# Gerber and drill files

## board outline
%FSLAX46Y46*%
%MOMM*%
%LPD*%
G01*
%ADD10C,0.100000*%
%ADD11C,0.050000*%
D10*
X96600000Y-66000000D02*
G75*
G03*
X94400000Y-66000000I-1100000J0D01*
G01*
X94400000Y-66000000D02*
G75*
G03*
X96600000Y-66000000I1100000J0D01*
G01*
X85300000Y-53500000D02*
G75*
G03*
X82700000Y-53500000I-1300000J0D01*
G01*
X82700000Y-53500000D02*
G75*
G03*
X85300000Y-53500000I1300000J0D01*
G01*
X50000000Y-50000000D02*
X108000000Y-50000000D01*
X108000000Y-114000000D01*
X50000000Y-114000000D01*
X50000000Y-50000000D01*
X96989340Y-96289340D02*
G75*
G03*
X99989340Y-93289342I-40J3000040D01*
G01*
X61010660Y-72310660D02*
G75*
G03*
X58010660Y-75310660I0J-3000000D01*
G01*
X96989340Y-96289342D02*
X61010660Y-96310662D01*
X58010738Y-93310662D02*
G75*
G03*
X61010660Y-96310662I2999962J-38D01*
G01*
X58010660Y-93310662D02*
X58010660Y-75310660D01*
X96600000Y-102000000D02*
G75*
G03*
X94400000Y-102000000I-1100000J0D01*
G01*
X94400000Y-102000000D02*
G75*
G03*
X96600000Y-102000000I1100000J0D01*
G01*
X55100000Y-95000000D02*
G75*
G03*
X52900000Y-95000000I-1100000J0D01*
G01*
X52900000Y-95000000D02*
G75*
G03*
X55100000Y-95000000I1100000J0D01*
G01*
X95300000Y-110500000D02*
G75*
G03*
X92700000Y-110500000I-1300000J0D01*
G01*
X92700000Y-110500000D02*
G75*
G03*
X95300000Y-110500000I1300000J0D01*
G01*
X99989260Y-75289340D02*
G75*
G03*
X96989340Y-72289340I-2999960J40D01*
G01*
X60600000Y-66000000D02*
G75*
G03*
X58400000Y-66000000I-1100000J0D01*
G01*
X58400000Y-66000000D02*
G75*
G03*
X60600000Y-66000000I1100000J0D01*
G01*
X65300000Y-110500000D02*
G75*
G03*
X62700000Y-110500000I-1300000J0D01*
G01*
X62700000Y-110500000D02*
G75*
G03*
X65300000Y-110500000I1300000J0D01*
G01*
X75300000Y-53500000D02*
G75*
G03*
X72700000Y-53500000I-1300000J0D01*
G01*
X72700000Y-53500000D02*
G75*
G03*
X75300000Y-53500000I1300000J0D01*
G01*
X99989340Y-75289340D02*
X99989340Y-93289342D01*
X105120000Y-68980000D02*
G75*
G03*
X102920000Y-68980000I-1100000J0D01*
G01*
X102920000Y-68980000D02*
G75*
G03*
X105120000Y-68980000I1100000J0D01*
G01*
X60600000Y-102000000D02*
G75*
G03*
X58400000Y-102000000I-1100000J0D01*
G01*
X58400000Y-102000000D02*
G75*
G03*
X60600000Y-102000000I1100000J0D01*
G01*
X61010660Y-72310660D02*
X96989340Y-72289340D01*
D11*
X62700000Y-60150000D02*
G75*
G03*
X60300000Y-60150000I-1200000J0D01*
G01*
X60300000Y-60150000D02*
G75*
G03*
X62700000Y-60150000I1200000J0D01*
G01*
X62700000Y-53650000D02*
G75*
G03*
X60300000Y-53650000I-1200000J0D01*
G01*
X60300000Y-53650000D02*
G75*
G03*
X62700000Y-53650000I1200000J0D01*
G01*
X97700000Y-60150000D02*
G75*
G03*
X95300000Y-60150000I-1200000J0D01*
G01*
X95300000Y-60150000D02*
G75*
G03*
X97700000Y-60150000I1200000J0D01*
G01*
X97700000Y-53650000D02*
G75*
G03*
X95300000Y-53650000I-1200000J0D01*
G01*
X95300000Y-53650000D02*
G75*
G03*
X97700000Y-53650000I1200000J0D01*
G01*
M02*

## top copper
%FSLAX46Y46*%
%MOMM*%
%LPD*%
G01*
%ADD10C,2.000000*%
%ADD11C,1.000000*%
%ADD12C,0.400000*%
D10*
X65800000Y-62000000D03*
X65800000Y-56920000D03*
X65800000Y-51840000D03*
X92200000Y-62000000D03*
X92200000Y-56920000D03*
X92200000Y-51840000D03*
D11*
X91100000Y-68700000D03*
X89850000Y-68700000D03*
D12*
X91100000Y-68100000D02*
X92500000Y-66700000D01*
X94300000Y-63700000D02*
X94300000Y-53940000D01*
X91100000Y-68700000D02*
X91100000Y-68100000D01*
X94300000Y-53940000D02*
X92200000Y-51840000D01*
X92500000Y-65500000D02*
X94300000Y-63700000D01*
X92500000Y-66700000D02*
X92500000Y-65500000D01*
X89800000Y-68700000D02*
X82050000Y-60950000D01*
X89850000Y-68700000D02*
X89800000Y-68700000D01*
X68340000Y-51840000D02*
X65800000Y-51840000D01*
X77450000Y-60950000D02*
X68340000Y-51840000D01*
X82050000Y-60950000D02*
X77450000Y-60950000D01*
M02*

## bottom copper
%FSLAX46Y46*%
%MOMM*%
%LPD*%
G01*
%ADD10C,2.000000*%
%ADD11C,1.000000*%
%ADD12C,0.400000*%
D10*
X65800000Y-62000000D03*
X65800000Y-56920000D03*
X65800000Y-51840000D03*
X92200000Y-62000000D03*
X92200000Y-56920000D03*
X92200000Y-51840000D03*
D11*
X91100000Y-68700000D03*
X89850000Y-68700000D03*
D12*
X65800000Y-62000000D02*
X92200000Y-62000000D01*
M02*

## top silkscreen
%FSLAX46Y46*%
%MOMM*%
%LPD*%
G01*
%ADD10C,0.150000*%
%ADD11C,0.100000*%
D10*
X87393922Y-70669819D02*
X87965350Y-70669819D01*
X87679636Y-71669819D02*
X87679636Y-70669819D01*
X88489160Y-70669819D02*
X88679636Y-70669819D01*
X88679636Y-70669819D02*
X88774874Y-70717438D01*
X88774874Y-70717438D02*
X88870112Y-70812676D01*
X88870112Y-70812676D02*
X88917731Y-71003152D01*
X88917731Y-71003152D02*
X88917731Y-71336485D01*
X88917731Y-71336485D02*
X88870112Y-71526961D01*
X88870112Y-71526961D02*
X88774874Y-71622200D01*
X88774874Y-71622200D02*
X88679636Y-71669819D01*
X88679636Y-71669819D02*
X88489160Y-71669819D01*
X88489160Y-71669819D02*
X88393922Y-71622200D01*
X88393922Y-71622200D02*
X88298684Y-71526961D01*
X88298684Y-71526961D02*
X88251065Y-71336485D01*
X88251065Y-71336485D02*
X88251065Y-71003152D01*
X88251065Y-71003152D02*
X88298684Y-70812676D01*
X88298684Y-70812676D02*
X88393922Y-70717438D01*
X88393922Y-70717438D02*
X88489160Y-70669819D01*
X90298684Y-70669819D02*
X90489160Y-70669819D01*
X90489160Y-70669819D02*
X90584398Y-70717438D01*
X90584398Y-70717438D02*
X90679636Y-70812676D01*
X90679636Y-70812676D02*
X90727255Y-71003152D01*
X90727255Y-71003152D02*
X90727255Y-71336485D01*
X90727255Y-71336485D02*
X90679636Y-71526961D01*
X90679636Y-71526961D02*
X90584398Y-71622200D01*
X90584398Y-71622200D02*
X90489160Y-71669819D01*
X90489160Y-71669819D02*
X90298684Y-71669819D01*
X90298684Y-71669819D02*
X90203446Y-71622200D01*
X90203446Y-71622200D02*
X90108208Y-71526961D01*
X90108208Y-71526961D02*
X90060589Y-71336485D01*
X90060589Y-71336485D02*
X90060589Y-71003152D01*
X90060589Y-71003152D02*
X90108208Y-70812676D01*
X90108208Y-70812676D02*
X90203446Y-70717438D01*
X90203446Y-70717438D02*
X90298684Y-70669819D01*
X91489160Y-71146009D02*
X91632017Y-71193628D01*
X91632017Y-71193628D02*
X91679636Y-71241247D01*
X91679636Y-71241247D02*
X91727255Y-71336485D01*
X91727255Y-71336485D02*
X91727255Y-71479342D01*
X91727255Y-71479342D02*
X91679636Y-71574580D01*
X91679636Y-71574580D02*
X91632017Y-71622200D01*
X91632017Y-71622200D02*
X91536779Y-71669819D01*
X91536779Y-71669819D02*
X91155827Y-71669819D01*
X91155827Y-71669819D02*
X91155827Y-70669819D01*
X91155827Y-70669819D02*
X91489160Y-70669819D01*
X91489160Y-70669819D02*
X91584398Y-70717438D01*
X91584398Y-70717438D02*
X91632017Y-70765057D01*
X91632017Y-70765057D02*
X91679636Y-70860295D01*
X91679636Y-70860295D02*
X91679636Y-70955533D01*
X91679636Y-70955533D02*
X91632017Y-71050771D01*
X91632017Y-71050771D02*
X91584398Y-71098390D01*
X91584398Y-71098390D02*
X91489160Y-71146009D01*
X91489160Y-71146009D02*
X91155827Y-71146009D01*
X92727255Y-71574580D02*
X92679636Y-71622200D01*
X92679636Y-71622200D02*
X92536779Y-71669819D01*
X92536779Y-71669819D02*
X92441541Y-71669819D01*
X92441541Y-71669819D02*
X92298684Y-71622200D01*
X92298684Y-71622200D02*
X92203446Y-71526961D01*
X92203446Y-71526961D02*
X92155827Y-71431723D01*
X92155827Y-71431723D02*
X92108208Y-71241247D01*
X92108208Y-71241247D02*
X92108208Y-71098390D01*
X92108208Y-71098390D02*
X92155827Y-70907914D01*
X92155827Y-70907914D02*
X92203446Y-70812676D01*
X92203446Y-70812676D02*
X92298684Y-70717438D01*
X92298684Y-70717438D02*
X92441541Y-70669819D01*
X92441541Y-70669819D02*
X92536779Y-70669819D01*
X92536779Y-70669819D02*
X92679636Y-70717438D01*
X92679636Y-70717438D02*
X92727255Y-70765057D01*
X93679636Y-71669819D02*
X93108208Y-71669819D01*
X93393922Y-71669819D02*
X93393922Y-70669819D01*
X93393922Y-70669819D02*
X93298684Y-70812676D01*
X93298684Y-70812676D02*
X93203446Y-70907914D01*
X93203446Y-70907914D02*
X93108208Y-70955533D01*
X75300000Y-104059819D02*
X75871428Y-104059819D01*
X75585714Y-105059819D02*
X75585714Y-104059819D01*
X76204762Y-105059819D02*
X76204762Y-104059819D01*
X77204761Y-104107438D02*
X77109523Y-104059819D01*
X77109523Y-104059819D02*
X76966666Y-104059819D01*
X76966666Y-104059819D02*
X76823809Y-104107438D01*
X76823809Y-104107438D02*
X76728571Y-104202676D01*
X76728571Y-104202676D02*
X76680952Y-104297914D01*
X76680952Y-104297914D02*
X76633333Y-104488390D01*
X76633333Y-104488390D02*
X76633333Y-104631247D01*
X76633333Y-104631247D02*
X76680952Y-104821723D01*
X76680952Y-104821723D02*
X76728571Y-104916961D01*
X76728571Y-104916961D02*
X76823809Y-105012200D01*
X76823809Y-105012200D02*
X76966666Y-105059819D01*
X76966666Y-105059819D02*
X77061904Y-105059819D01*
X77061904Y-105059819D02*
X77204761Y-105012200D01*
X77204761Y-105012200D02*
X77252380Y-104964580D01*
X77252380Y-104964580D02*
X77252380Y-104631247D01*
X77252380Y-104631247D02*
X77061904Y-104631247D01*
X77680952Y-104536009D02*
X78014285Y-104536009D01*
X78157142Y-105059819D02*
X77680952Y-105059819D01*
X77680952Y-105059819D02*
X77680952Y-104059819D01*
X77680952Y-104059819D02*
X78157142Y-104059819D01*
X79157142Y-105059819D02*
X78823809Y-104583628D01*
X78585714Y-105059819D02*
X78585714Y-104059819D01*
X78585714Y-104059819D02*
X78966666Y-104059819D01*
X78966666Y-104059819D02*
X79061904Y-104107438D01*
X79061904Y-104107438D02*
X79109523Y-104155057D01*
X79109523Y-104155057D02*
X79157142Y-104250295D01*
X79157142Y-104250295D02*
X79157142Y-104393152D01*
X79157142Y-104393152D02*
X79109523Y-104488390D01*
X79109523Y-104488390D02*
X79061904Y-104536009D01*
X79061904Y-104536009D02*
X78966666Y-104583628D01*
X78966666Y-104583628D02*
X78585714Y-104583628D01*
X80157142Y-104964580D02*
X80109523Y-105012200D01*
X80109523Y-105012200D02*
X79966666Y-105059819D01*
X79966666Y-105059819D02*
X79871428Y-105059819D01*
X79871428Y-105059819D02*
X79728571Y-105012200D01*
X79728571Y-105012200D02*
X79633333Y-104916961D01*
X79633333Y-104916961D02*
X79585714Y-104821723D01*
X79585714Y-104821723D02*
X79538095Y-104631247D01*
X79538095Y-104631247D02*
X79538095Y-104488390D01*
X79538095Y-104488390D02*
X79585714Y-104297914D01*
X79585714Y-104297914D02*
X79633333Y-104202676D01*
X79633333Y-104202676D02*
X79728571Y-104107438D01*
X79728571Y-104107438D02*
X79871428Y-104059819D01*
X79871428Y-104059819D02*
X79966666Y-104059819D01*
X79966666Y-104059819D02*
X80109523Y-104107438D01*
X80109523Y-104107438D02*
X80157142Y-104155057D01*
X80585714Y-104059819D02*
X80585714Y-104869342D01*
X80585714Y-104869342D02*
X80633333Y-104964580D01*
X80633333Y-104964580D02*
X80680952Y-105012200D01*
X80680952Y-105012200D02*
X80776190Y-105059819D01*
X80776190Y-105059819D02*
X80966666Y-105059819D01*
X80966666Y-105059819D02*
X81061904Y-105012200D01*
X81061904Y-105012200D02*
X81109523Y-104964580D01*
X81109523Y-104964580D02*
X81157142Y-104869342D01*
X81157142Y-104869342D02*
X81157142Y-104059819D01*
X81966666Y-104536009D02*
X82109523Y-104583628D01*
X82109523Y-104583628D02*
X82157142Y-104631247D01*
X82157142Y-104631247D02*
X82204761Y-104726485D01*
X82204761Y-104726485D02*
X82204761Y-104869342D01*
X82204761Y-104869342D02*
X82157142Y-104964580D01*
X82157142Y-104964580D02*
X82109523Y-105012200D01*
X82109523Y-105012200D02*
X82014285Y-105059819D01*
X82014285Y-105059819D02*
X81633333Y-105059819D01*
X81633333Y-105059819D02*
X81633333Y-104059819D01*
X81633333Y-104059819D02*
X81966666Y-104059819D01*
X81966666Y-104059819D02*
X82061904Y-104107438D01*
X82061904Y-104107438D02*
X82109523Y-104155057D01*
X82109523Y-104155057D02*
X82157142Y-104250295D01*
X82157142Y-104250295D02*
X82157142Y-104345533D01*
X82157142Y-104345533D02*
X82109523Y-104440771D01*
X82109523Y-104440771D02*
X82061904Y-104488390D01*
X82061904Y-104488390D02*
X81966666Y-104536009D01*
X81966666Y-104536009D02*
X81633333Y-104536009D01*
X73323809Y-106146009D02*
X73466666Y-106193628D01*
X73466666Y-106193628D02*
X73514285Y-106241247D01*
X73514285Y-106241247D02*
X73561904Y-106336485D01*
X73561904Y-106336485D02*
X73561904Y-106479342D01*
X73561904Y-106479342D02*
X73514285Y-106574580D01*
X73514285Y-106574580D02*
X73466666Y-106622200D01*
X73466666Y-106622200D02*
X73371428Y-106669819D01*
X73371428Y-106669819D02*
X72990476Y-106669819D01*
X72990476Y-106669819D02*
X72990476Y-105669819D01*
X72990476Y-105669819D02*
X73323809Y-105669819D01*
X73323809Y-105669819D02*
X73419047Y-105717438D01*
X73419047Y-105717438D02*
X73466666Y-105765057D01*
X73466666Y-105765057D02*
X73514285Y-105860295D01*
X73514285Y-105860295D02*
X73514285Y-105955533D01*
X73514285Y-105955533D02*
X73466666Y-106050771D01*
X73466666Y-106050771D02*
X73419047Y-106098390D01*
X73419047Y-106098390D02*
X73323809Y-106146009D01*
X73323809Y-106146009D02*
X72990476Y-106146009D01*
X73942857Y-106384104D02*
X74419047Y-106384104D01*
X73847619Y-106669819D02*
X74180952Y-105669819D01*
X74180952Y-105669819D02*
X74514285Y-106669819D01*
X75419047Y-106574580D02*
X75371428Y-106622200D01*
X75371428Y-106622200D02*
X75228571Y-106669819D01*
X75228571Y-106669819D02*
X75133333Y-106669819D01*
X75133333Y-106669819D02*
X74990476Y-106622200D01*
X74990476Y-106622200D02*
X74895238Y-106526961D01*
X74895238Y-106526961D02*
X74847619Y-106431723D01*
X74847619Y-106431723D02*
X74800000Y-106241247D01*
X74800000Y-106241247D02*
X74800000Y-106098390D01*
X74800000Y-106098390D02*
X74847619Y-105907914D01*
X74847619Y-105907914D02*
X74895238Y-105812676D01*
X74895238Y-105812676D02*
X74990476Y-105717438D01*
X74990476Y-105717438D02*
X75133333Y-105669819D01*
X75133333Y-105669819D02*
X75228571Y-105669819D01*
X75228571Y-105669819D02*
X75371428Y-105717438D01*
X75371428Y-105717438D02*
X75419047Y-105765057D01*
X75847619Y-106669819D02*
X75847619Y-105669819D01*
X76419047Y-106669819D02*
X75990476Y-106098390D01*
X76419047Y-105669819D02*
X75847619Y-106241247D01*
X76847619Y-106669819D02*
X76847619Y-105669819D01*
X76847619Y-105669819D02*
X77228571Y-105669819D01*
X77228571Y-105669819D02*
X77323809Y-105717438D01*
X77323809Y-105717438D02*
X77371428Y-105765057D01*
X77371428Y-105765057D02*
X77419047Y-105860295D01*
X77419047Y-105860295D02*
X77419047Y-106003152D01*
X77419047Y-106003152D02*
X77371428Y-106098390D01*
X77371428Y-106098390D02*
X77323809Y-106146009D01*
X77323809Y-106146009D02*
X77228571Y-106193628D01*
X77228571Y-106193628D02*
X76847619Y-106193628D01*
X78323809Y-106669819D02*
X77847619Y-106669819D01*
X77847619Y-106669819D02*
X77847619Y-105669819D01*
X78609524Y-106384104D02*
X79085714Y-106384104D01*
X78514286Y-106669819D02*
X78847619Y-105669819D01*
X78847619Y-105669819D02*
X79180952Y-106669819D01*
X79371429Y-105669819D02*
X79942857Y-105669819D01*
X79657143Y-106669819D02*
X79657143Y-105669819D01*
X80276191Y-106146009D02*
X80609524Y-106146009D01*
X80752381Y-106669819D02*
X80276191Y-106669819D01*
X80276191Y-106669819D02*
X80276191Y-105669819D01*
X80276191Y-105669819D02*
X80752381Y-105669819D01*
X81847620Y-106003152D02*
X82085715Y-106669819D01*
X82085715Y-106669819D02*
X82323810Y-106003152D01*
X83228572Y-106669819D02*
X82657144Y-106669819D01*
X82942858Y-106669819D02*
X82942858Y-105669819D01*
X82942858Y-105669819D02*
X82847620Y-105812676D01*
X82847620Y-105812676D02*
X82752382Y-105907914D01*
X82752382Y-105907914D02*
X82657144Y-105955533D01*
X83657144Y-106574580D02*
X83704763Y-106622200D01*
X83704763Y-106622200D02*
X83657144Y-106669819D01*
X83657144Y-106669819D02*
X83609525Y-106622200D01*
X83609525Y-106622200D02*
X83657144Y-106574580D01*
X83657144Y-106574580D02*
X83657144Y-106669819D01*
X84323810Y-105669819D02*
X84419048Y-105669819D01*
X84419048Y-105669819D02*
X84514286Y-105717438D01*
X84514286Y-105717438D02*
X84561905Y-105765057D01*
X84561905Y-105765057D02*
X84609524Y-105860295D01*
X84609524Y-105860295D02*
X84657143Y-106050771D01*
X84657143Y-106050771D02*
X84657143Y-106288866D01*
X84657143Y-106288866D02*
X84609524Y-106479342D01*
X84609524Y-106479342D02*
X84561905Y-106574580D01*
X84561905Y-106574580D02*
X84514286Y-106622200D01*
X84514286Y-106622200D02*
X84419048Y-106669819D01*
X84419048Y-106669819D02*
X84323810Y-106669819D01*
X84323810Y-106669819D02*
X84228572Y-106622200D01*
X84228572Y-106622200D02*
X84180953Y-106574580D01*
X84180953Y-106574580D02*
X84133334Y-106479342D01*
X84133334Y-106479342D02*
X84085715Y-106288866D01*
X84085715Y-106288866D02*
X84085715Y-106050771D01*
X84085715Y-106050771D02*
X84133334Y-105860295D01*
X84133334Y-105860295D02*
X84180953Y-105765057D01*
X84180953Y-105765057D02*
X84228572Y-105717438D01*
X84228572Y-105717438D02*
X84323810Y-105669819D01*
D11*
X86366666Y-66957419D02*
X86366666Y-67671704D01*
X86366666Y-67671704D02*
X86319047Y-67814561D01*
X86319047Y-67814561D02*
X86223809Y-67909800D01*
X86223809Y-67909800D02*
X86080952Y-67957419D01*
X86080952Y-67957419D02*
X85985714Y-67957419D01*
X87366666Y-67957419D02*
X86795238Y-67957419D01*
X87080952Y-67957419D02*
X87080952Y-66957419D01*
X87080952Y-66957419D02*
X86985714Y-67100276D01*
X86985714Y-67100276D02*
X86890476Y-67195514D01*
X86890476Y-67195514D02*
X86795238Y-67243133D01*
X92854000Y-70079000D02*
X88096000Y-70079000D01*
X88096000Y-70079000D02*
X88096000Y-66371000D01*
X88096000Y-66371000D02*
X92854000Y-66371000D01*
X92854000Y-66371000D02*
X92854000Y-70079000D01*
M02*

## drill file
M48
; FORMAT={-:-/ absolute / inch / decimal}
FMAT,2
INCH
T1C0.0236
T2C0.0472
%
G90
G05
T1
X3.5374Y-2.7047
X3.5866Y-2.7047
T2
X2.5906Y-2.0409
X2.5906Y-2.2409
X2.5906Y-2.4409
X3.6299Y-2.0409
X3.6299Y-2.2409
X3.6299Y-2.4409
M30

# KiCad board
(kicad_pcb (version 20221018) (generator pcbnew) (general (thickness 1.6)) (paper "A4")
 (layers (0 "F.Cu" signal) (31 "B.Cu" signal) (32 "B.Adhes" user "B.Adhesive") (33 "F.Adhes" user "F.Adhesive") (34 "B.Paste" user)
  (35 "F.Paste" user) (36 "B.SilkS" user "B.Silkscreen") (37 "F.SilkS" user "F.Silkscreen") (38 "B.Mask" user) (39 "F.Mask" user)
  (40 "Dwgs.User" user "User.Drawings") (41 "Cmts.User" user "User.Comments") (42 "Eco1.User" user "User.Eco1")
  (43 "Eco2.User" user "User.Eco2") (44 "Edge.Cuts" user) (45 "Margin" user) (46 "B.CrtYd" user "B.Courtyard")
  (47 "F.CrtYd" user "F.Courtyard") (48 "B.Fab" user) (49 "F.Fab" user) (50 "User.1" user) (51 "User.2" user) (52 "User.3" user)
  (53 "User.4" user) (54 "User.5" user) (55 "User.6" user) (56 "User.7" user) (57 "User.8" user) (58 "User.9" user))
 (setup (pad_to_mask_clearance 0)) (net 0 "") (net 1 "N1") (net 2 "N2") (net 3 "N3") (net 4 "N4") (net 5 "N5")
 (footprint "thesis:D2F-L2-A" (layer "F.Cu") (at 55.865 63.835 90)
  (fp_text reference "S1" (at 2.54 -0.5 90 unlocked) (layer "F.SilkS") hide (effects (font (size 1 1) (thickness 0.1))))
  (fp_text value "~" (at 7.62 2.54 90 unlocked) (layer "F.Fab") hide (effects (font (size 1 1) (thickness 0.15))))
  (fp_circle (center 3.685 5.635) (end 4.885 5.635) (stroke (width 0.05) (type default)) (fill none) (layer "Edge.Cuts"))
  (fp_circle (center 10.185 5.635) (end 11.385 5.635) (stroke (width 0.05) (type default)) (fill none) (layer "Edge.Cuts"))
  (pad "1" thru_hole circle (at 1.835 9.935 90) (size 2 2) (drill 1.2) (layers "*.Cu" "*.Mask") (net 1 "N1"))
  (pad "2" thru_hole circle (at 6.915 9.935 90) (size 2 2) (drill 1.2) (layers "*.Cu" "*.Mask") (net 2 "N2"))
  (pad "3" thru_hole circle (at 11.995 9.935 90) (size 2 2) (drill 1.2) (layers "*.Cu" "*.Mask") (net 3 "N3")))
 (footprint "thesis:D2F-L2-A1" (layer "F.Cu") (at 94.365 63.835 90)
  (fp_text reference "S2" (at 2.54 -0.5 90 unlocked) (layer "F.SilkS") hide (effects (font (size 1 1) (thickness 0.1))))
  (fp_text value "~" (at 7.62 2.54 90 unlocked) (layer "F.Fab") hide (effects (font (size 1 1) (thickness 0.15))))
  (fp_circle (center 3.685 2.135) (end 4.885 2.135) (stroke (width 0.05) (type default)) (fill none) (layer "Edge.Cuts"))
  (fp_circle (center 10.185 2.135) (end 11.385 2.135) (stroke (width 0.05) (type default)) (fill none) (layer "Edge.Cuts"))
  (pad "1" thru_hole circle (at 1.835 -2.165 90) (size 2 2) (drill 1.2) (layers "*.Cu" "*.Mask") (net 1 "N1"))
  (pad "2" thru_hole circle (at 6.915 -2.165 90) (size 2 2) (drill 1.2) (layers "*.Cu" "*.Mask") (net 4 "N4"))
  (pad "3" thru_hole circle (at 11.995 -2.165 90) (size 2 2) (drill 1.2) (layers "*.Cu" "*.Mask") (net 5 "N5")))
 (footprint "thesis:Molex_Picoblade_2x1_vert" (layer "F.Cu") (at 92.6 69.97 180)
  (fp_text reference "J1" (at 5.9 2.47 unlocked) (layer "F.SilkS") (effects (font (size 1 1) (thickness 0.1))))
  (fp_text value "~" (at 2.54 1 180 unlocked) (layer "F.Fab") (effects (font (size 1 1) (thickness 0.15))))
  (fp_rect (start -0.254 -0.109) (end 4.504 3.599) (stroke (width 0.1) (type default)) (fill none) (layer "F.SilkS"))
  (pad "1" thru_hole circle (at 1.5 1.27 180) (size 1 1) (drill 0.6) (layers "*.Cu" "*.Mask") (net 5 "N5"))
  (pad "2" thru_hole circle (at 2.75 1.27 180) (size 1 1) (drill 0.6) (layers "*.Cu" "*.Mask") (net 3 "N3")))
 (gr_circle (center 95.5 66) (end 96.6 66) (stroke (width 0.1) (type default)) (fill none) (layer "Edge.Cuts"))
 (gr_circle (center 84 53.5) (end 85.3 53.5) (stroke (width 0.1) (type default)) (fill none) (layer "Edge.Cuts"))
 (gr_rect (start 50 50) (end 108 114) (stroke (width 0.1) (type default)) (fill none) (layer "Edge.Cuts"))
 (gr_arc (start 99.98934 93.289342) (mid 99.11066 95.410662) (end 96.98934 96.289342) (stroke (width 0.1) (type default))
  (layer "Edge.Cuts"))
 (gr_arc (start 58.01066 75.31066) (mid 58.88934 73.18934) (end 61.01066 72.31066) (stroke (width 0.1) (type default)) (layer "Edge.Cuts"))
 (gr_line (start 96.98934 96.289342) (end 61.01066 96.310662) (stroke (width 0.1) (type default)) (layer "Edge.Cuts"))
 (gr_arc (start 61.01066 96.310662) (mid 58.88934 95.431982) (end 58.01066 93.310662) (stroke (width 0.1) (type default))
  (layer "Edge.Cuts"))
 (gr_line (start 58.01066 93.310662) (end 58.01066 75.31066) (stroke (width 0.1) (type default)) (layer "Edge.Cuts"))
 (gr_circle (center 95.5 102) (end 96.6 102) (stroke (width 0.1) (type default)) (fill none) (layer "Edge.Cuts"))
 (gr_circle (center 54 95) (end 55.1 95) (stroke (width 0.1) (type default)) (fill none) (layer "Edge.Cuts"))
 (gr_circle (center 94 110.5) (end 95.3 110.5) (stroke (width 0.1) (type default)) (fill none) (layer "Edge.Cuts"))
 (gr_arc (start 96.98934 72.28934) (mid 99.11066 73.16802) (end 99.98934 75.28934) (stroke (width 0.1) (type default)) (layer "Edge.Cuts"))
 (gr_circle (center 59.5 66) (end 60.6 66) (stroke (width 0.1) (type default)) (fill none) (layer "Edge.Cuts"))
 (gr_circle (center 64 110.5) (end 65.3 110.5) (stroke (width 0.1) (type default)) (fill none) (layer "Edge.Cuts"))
 (gr_circle (center 74 53.5) (end 75.3 53.5) (stroke (width 0.1) (type default)) (fill none) (layer "Edge.Cuts"))
 (gr_line (start 99.98934 75.28934) (end 99.98934 93.289342) (stroke (width 0.1) (type default)) (layer "Edge.Cuts"))
 (gr_circle (center 104.02 68.98) (end 105.12 68.98) (stroke (width 0.1) (type default)) (fill none) (layer "Edge.Cuts"))
 (gr_circle (center 59.5 102) (end 60.6 102) (stroke (width 0.1) (type default)) (fill none) (layer "Edge.Cuts"))
 (gr_line (start 61.01066 72.31066) (end 96.98934 72.28934) (stroke (width 0.1) (type default)) (layer "Edge.Cuts"))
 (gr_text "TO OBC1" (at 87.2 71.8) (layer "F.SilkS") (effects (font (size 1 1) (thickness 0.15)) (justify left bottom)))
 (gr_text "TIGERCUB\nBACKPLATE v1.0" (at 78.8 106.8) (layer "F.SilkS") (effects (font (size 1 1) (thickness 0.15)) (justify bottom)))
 (segment (start 91.1 68.1) (end 92.5 66.7) (width 0.4) (layer "F.Cu") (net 5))
 (segment (start 94.3 63.7) (end 94.3 53.94) (width 0.4) (layer "F.Cu") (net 5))
 (segment (start 91.1 68.7) (end 91.1 68.1) (width 0.4) (layer "F.Cu") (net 5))
 (segment (start 94.3 53.94) (end 92.2 51.84) (width 0.4) (layer "F.Cu") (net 5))
 (segment (start 92.5 65.5) (end 94.3 63.7) (width 0.4) (layer "F.Cu") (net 5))
 (segment (start 92.5 66.7) (end 92.5 65.5) (width 0.4) (layer "F.Cu") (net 5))
 (segment (start 89.8 68.7) (end 82.05 60.95) (width 0.4) (layer "F.Cu") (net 3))
 (segment (start 89.85 68.7) (end 89.8 68.7) (width 0.4) (layer "F.Cu") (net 3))
 (segment (start 68.34 51.84) (end 65.8 51.84) (width 0.4) (layer "F.Cu") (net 3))
 (segment (start 77.45 60.95) (end 68.34 51.84) (width 0.4) (layer "F.Cu") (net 3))
 (segment (start 82.05 60.95) (end 77.45 60.95) (width 0.4) (layer "F.Cu") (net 3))
 (segment (start 65.8 62) (end 92.2 62) (width 0.4) (layer "B.Cu") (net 1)))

